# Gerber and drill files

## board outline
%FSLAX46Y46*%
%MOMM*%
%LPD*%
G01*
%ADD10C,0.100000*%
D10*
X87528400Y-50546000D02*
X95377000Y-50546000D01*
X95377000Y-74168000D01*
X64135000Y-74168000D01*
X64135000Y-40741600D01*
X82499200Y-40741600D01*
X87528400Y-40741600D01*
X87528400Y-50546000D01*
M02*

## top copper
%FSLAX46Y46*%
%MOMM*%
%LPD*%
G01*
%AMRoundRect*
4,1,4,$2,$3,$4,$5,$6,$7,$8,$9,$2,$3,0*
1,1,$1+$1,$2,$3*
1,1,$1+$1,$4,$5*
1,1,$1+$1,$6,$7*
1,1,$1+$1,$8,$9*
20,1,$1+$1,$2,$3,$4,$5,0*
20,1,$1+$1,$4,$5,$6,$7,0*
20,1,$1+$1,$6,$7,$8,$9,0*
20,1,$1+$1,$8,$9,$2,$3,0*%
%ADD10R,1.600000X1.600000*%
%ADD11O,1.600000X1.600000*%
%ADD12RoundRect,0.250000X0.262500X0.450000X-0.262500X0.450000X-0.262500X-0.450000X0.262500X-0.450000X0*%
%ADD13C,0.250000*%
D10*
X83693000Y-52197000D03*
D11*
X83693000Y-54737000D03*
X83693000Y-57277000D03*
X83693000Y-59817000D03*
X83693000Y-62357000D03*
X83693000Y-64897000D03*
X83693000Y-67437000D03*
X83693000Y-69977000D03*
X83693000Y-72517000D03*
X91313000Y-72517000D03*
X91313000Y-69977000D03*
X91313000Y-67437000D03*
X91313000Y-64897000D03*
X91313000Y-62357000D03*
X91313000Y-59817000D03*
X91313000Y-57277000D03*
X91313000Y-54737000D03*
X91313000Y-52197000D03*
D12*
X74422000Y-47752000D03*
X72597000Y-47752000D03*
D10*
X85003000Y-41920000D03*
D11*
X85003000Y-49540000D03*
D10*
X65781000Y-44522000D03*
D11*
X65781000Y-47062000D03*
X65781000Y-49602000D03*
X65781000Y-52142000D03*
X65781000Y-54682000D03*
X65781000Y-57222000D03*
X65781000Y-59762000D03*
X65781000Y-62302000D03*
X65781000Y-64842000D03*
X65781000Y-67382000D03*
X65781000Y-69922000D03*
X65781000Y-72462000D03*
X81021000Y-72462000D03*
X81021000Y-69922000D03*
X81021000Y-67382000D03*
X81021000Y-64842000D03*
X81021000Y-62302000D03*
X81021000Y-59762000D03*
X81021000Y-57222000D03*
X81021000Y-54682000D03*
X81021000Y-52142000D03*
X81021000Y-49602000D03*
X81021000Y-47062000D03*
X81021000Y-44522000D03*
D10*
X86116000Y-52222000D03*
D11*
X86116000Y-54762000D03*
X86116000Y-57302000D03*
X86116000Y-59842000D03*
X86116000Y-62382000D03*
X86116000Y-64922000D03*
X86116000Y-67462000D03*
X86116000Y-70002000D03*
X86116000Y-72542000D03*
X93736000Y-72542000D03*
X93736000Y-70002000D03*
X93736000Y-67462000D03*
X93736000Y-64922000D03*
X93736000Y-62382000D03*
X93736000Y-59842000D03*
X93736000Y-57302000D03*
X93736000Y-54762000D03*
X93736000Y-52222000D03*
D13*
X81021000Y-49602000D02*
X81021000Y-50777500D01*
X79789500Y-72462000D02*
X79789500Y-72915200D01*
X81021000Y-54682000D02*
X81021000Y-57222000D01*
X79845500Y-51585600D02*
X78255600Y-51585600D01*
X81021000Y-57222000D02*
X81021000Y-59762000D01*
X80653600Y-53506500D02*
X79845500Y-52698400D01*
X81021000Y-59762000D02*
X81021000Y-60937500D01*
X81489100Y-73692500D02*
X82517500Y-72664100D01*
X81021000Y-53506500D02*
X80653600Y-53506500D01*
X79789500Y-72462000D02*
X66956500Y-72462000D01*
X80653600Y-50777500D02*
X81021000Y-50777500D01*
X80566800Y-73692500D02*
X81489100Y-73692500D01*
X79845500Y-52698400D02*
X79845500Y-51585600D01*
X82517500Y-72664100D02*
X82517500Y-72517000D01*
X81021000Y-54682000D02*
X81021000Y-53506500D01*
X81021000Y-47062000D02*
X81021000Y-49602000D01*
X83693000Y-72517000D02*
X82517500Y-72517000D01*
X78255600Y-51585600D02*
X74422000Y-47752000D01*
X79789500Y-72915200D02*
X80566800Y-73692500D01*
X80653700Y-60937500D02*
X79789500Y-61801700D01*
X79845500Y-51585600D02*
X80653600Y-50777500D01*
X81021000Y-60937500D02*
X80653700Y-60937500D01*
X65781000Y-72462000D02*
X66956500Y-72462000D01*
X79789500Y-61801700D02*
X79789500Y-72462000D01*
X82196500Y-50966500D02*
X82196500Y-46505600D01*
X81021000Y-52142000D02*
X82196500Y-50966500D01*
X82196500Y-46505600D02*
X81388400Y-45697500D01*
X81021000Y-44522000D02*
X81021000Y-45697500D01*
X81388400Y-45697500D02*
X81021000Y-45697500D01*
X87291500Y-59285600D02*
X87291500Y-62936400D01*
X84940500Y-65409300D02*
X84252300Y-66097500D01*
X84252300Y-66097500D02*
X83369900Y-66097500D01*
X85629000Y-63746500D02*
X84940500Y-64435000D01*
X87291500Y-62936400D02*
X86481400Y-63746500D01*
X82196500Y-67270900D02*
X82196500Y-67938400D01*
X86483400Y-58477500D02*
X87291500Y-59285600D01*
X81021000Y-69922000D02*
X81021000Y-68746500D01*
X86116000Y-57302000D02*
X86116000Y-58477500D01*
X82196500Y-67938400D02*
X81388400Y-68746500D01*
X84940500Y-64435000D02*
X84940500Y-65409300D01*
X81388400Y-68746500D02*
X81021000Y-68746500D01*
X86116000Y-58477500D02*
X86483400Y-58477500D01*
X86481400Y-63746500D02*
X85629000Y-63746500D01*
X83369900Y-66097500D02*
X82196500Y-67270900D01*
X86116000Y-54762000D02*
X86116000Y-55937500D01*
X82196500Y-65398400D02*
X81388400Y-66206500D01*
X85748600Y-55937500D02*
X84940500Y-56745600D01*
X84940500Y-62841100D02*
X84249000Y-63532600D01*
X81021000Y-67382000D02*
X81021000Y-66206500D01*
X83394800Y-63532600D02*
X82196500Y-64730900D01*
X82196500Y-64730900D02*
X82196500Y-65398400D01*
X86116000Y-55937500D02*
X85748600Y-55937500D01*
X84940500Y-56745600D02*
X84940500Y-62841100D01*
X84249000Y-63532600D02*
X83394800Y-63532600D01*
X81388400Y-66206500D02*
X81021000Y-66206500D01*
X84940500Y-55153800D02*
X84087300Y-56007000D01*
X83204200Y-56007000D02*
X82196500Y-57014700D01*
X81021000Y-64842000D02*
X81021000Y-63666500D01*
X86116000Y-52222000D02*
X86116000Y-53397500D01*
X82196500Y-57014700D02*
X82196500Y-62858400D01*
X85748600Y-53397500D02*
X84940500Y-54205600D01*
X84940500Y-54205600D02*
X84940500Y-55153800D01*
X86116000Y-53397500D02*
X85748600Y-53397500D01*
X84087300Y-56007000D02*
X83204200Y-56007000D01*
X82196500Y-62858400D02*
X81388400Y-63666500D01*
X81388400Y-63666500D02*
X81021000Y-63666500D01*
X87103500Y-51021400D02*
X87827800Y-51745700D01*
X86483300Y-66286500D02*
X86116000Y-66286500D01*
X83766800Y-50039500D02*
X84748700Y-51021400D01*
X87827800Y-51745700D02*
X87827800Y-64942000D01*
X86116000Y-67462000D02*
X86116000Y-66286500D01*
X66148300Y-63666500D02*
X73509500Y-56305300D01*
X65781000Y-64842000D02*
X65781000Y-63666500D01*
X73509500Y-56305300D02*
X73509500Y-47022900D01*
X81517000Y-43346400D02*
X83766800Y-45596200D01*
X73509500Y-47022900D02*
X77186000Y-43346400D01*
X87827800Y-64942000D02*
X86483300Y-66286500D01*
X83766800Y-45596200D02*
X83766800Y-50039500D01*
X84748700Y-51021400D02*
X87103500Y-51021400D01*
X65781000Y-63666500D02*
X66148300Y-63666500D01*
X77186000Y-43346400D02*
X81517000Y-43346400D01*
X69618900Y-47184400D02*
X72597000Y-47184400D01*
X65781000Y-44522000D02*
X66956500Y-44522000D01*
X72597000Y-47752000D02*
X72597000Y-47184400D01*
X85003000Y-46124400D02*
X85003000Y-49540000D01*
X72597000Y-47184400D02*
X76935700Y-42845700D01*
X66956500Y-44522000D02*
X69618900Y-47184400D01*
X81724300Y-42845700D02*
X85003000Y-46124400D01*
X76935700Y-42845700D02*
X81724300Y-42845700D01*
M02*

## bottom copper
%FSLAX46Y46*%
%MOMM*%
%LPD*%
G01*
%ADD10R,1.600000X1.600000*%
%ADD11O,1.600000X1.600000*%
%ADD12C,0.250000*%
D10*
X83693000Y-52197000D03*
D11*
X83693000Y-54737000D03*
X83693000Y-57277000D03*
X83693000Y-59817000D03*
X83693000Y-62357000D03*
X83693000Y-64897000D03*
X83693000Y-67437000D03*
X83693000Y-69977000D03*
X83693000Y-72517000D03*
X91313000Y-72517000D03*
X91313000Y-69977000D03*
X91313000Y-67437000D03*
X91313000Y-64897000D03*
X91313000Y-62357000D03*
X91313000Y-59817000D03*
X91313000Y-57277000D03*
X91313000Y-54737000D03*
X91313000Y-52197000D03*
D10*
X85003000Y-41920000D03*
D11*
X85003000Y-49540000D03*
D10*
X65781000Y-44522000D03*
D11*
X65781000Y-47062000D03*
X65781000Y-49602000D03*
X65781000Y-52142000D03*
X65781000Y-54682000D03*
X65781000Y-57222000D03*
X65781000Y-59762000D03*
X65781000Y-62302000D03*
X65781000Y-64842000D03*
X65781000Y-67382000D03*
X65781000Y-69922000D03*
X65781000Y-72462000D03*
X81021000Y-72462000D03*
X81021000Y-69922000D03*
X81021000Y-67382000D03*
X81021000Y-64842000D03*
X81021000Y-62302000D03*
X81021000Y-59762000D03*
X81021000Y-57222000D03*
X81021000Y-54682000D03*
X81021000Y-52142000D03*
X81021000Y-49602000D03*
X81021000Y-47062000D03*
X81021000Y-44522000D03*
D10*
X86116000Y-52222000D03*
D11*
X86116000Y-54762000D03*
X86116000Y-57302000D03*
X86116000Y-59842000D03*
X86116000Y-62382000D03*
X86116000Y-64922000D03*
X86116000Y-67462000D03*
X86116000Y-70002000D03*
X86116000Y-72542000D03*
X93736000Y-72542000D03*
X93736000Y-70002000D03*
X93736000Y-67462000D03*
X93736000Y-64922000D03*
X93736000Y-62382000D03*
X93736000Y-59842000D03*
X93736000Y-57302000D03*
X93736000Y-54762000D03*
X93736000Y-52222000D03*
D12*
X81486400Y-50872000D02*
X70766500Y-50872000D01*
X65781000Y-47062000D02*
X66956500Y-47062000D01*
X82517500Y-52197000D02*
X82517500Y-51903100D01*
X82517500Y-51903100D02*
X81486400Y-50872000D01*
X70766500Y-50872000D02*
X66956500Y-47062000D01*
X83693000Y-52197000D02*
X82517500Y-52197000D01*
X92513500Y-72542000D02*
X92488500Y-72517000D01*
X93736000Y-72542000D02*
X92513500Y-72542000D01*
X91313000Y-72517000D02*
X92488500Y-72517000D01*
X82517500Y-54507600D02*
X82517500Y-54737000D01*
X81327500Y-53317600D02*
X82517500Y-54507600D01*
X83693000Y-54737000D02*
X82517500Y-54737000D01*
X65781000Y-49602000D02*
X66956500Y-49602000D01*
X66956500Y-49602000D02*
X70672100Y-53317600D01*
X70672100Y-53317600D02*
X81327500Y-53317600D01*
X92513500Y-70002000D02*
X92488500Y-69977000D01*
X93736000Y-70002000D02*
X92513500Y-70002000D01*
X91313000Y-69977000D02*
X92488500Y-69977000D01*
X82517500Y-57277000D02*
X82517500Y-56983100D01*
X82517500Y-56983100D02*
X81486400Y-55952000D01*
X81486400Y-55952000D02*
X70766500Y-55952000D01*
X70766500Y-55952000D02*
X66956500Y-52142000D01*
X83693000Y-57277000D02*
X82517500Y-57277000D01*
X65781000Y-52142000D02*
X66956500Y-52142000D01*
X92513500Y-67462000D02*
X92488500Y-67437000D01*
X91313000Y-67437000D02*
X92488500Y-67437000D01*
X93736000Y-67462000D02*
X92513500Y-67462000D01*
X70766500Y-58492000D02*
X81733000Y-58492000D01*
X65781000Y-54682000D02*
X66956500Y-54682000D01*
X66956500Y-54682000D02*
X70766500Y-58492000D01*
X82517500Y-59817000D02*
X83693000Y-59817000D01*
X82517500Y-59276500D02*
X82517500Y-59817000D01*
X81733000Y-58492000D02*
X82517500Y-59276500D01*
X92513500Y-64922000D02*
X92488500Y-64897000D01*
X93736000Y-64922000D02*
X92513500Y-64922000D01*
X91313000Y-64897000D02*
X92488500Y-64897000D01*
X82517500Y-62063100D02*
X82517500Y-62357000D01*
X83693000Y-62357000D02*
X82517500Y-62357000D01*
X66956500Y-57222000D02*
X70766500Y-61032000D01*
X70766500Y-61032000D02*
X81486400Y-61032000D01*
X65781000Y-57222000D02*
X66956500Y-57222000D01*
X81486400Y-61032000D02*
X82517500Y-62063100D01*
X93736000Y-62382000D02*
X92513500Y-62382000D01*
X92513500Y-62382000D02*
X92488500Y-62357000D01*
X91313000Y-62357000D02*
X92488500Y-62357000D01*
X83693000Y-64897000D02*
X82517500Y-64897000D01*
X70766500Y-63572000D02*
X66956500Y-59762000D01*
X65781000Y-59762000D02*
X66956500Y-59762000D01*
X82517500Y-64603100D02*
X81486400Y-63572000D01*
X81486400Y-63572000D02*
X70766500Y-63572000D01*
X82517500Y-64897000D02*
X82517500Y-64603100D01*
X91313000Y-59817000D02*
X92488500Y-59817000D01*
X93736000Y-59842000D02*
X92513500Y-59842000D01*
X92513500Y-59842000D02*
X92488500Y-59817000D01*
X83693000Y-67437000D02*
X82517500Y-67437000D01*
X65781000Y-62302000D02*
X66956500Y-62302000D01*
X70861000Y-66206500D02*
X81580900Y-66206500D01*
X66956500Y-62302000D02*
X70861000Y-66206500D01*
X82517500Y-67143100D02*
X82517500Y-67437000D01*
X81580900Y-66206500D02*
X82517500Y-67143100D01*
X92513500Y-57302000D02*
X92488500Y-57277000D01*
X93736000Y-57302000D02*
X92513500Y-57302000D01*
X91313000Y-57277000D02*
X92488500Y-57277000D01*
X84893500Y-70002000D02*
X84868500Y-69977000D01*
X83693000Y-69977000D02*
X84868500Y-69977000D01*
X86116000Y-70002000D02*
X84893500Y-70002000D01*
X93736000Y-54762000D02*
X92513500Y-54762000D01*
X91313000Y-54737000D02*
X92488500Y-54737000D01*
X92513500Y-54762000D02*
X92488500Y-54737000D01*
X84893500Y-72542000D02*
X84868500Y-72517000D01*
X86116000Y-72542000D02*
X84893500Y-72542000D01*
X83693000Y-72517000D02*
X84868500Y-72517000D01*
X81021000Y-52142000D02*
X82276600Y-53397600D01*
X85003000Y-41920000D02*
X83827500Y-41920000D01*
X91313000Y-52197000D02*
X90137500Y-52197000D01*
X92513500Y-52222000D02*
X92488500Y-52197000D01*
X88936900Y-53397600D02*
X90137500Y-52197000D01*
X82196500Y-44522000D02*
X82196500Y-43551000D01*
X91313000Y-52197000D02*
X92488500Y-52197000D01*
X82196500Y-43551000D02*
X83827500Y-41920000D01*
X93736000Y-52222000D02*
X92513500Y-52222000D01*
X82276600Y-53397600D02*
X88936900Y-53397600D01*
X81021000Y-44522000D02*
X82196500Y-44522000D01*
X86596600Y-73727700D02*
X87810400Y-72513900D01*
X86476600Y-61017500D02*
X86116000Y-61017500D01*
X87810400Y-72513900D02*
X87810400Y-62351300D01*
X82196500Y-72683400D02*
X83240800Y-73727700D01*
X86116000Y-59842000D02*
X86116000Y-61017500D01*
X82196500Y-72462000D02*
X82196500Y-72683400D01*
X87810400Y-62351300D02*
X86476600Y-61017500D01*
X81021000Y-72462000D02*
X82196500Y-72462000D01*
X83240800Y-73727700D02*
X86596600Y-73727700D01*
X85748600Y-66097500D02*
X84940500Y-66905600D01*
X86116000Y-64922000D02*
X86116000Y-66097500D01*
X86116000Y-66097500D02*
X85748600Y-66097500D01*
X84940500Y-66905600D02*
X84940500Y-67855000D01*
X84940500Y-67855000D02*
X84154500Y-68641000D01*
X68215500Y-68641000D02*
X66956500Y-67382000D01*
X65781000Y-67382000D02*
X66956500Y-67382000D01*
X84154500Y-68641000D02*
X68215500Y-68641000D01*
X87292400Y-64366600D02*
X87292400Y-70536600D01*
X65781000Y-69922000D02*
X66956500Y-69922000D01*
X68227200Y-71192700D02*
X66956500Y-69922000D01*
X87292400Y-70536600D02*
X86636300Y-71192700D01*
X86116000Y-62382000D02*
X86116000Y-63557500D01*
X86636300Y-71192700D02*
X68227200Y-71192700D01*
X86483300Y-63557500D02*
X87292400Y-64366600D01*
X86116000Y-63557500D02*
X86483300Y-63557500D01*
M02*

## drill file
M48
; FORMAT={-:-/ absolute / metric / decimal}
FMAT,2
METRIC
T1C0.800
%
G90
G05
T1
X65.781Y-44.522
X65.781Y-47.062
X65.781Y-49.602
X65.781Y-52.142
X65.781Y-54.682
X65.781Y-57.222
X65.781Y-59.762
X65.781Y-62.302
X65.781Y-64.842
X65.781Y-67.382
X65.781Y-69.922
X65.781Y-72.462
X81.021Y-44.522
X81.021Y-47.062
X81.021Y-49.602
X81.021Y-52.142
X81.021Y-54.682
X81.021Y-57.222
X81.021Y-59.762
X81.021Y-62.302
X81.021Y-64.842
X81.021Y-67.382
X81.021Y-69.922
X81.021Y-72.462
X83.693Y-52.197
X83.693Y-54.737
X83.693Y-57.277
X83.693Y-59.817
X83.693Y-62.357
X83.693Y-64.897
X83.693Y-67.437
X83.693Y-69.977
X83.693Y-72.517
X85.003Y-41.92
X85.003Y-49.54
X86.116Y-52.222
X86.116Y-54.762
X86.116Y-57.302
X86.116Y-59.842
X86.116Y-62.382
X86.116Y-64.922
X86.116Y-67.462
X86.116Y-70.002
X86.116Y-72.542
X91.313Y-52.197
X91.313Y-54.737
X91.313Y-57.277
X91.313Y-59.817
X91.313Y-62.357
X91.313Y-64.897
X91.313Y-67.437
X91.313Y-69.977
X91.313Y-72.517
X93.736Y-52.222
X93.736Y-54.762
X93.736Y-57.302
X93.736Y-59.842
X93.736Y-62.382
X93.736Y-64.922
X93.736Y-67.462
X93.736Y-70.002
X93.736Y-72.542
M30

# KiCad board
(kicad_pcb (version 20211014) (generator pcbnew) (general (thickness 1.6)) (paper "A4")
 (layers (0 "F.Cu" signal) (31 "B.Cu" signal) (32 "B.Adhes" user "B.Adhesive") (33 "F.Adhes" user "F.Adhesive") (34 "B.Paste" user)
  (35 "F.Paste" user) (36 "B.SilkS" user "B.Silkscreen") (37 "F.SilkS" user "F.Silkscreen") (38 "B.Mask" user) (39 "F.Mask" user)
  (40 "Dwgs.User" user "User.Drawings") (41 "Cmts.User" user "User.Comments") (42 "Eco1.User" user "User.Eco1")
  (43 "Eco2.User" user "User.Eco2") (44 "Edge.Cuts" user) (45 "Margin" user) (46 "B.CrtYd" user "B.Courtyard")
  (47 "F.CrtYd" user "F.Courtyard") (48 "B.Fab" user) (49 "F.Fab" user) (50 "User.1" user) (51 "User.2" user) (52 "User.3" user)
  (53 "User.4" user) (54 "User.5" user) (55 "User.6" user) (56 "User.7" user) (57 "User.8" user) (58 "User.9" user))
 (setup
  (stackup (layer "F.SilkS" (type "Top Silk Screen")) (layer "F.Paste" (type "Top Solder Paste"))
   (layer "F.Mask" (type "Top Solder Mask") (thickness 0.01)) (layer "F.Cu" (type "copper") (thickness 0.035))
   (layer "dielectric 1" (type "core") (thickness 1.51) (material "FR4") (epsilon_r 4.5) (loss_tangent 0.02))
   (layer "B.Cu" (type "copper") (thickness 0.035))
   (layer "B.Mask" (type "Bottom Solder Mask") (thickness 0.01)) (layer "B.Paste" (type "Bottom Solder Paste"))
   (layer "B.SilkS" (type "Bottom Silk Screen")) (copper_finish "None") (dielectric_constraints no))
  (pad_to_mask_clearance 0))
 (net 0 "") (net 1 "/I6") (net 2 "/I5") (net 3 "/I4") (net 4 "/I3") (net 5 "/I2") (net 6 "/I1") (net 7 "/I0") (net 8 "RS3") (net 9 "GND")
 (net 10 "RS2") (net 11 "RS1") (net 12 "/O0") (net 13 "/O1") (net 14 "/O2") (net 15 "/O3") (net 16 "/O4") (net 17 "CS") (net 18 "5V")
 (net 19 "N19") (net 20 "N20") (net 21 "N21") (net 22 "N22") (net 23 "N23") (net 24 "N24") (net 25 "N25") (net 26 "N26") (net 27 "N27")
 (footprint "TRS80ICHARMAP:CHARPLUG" (layer "F.Cu") (at 83.693 52.197)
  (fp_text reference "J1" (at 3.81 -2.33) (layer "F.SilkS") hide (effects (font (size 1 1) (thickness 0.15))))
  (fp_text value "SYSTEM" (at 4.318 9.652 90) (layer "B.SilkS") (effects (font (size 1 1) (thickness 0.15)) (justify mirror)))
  (pad "1" thru_hole rect (at 0 0) (size 1.6 1.6) (drill 0.8) (layers *.Cu *.Mask) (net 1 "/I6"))
  (pad "2" thru_hole oval (at 0 2.54) (size 1.6 1.6) (drill 0.8) (layers *.Cu *.Mask) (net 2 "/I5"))
  (pad "3" thru_hole oval (at 0 5.08) (size 1.6 1.6) (drill 0.8) (layers *.Cu *.Mask) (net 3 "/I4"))
  (pad "4" thru_hole oval (at 0 7.62) (size 1.6 1.6) (drill 0.8) (layers *.Cu *.Mask) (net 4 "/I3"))
  (pad "5" thru_hole oval (at 0 10.16) (size 1.6 1.6) (drill 0.8) (layers *.Cu *.Mask) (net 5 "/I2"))
  (pad "6" thru_hole oval (at 0 12.7) (size 1.6 1.6) (drill 0.8) (layers *.Cu *.Mask) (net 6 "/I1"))
  (pad "7" thru_hole oval (at 0 15.24) (size 1.6 1.6) (drill 0.8) (layers *.Cu *.Mask) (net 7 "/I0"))
  (pad "8" thru_hole oval (at 0 17.78) (size 1.6 1.6) (drill 0.8) (layers *.Cu *.Mask) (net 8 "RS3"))
  (pad "9" thru_hole oval (at 0 20.32) (size 1.6 1.6) (drill 0.8) (layers *.Cu *.Mask) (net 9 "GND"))
  (pad "10" thru_hole oval (at 7.62 20.32) (size 1.6 1.6) (drill 0.8) (layers *.Cu *.Mask) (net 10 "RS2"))
  (pad "11" thru_hole oval (at 7.62 17.78) (size 1.6 1.6) (drill 0.8) (layers *.Cu *.Mask) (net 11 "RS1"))
  (pad "12" thru_hole oval (at 7.62 15.24) (size 1.6 1.6) (drill 0.8) (layers *.Cu *.Mask) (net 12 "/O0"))
  (pad "13" thru_hole oval (at 7.62 12.7) (size 1.6 1.6) (drill 0.8) (layers *.Cu *.Mask) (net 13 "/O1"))
  (pad "14" thru_hole oval (at 7.62 10.16) (size 1.6 1.6) (drill 0.8) (layers *.Cu *.Mask) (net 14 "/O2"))
  (pad "15" thru_hole oval (at 7.62 7.62) (size 1.6 1.6) (drill 0.8) (layers *.Cu *.Mask) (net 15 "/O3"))
  (pad "16" thru_hole oval (at 7.62 5.08) (size 1.6 1.6) (drill 0.8) (layers *.Cu *.Mask) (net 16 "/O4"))
  (pad "17" thru_hole oval (at 7.62 2.54) (size 1.6 1.6) (drill 0.8) (layers *.Cu *.Mask) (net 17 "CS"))
  (pad "18" thru_hole oval (at 7.62 0) (size 1.6 1.6) (drill 0.8) (layers *.Cu *.Mask) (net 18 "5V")))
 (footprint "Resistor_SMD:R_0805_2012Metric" (layer "F.Cu") (at 73.5095 47.752 180)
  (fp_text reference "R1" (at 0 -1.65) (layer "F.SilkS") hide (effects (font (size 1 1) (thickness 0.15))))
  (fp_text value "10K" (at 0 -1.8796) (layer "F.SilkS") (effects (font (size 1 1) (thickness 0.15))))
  (pad "1" smd roundrect locked (at -0.9125 0 180) (size 1.025 1.4) (layers "F.Cu" "F.Paste" "F.Mask") (roundrect_rratio 0.243902439)
   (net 9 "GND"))
  (pad "2" smd roundrect locked (at 0.9125 0 180) (size 1.025 1.4) (layers "F.Cu" "F.Paste" "F.Mask") (roundrect_rratio 0.243902439)
   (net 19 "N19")))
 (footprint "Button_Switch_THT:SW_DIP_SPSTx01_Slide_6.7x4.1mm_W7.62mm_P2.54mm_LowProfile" (layer "F.Cu") (at 85.003 41.92 -90)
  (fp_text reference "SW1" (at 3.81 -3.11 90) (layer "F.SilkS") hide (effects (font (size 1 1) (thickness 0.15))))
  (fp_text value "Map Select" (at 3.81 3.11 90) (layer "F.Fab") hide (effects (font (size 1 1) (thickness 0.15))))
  (pad "1" thru_hole rect locked (at 0 0 270) (size 1.6 1.6) (drill 0.8) (layers *.Cu *.Mask) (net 18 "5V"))
  (pad "2" thru_hole oval locked (at 7.62 0 270) (size 1.6 1.6) (drill 0.8) (layers *.Cu *.Mask) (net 19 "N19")))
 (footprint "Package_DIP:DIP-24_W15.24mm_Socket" (layer "F.Cu") (at 65.781 44.522)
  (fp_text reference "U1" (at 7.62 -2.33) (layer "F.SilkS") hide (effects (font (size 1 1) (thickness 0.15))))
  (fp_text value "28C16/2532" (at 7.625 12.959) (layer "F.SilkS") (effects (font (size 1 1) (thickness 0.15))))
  (pad "1" thru_hole rect locked (at 0 0) (size 1.6 1.6) (drill 0.8) (layers *.Cu *.Mask) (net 19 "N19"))
  (pad "2" thru_hole oval locked (at 0 2.54) (size 1.6 1.6) (drill 0.8) (layers *.Cu *.Mask) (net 1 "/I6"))
  (pad "3" thru_hole oval locked (at 0 5.08) (size 1.6 1.6) (drill 0.8) (layers *.Cu *.Mask) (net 2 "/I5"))
  (pad "4" thru_hole oval locked (at 0 7.62) (size 1.6 1.6) (drill 0.8) (layers *.Cu *.Mask) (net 3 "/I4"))
  (pad "5" thru_hole oval locked (at 0 10.16) (size 1.6 1.6) (drill 0.8) (layers *.Cu *.Mask) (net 4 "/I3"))
  (pad "6" thru_hole oval locked (at 0 12.7) (size 1.6 1.6) (drill 0.8) (layers *.Cu *.Mask) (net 5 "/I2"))
  (pad "7" thru_hole oval locked (at 0 15.24) (size 1.6 1.6) (drill 0.8) (layers *.Cu *.Mask) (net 6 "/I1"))
  (pad "8" thru_hole oval locked (at 0 17.78) (size 1.6 1.6) (drill 0.8) (layers *.Cu *.Mask) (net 7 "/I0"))
  (pad "9" thru_hole oval locked (at 0 20.32) (size 1.6 1.6) (drill 0.8) (layers *.Cu *.Mask) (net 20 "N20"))
  (pad "10" thru_hole oval locked (at 0 22.86) (size 1.6 1.6) (drill 0.8) (layers *.Cu *.Mask) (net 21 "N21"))
  (pad "11" thru_hole oval locked (at 0 25.4) (size 1.6 1.6) (drill 0.8) (layers *.Cu *.Mask) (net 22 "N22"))
  (pad "12" thru_hole oval locked (at 0 27.94) (size 1.6 1.6) (drill 0.8) (layers *.Cu *.Mask) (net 9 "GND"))
  (pad "13" thru_hole oval locked (at 15.24 27.94) (size 1.6 1.6) (drill 0.8) (layers *.Cu *.Mask) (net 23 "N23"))
  (pad "14" thru_hole oval locked (at 15.24 25.4) (size 1.6 1.6) (drill 0.8) (layers *.Cu *.Mask) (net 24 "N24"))
  (pad "15" thru_hole oval locked (at 15.24 22.86) (size 1.6 1.6) (drill 0.8) (layers *.Cu *.Mask) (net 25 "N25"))
  (pad "16" thru_hole oval locked (at 15.24 20.32) (size 1.6 1.6) (drill 0.8) (layers *.Cu *.Mask) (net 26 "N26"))
  (pad "17" thru_hole oval locked (at 15.24 17.78) (size 1.6 1.6) (drill 0.8) (layers *.Cu *.Mask) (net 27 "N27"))
  (pad "18" thru_hole oval locked (at 15.24 15.24) (size 1.6 1.6) (drill 0.8) (layers *.Cu *.Mask) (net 9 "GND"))
  (pad "19" thru_hole oval locked (at 15.24 12.7) (size 1.6 1.6) (drill 0.8) (layers *.Cu *.Mask) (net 9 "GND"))
  (pad "20" thru_hole oval locked (at 15.24 10.16) (size 1.6 1.6) (drill 0.8) (layers *.Cu *.Mask) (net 9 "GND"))
  (pad "21" thru_hole oval locked (at 15.24 7.62) (size 1.6 1.6) (drill 0.8) (layers *.Cu *.Mask) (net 18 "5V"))
  (pad "22" thru_hole oval locked (at 15.24 5.08) (size 1.6 1.6) (drill 0.8) (layers *.Cu *.Mask) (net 9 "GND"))
  (pad "23" thru_hole oval locked (at 15.24 2.54) (size 1.6 1.6) (drill 0.8) (layers *.Cu *.Mask) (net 9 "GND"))
  (pad "24" thru_hole oval locked (at 15.24 0) (size 1.6 1.6) (drill 0.8) (layers *.Cu *.Mask) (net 18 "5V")))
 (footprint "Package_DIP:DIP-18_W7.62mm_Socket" (layer "F.Cu") (at 86.116 52.222)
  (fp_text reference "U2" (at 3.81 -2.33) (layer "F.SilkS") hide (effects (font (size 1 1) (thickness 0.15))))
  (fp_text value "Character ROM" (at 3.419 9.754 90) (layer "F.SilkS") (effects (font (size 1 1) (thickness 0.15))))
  (pad "1" thru_hole rect locked (at 0 0) (size 1.6 1.6) (drill 0.8) (layers *.Cu *.Mask) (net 26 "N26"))
  (pad "2" thru_hole oval locked (at 0 2.54) (size 1.6 1.6) (drill 0.8) (layers *.Cu *.Mask) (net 25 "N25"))
  (pad "3" thru_hole oval locked (at 0 5.08) (size 1.6 1.6) (drill 0.8) (layers *.Cu *.Mask) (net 24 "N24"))
  (pad "4" thru_hole oval locked (at 0 7.62) (size 1.6 1.6) (drill 0.8) (layers *.Cu *.Mask) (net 23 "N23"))
  (pad "5" thru_hole oval locked (at 0 10.16) (size 1.6 1.6) (drill 0.8) (layers *.Cu *.Mask) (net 22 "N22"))
  (pad "6" thru_hole oval locked (at 0 12.7) (size 1.6 1.6) (drill 0.8) (layers *.Cu *.Mask) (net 21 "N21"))
  (pad "7" thru_hole oval locked (at 0 15.24) (size 1.6 1.6) (drill 0.8) (layers *.Cu *.Mask) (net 20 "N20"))
  (pad "8" thru_hole oval locked (at 0 17.78) (size 1.6 1.6) (drill 0.8) (layers *.Cu *.Mask) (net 8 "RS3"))
  (pad "9" thru_hole oval locked (at 0 20.32) (size 1.6 1.6) (drill 0.8) (layers *.Cu *.Mask) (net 9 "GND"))
  (pad "10" thru_hole oval locked (at 7.62 20.32) (size 1.6 1.6) (drill 0.8) (layers *.Cu *.Mask) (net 10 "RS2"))
  (pad "11" thru_hole oval locked (at 7.62 17.78) (size 1.6 1.6) (drill 0.8) (layers *.Cu *.Mask) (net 11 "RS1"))
  (pad "12" thru_hole oval locked (at 7.62 15.24) (size 1.6 1.6) (drill 0.8) (layers *.Cu *.Mask) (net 12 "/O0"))
  (pad "13" thru_hole oval locked (at 7.62 12.7) (size 1.6 1.6) (drill 0.8) (layers *.Cu *.Mask) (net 13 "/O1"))
  (pad "14" thru_hole oval locked (at 7.62 10.16) (size 1.6 1.6) (drill 0.8) (layers *.Cu *.Mask) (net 14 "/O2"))
  (pad "15" thru_hole oval locked (at 7.62 7.62) (size 1.6 1.6) (drill 0.8) (layers *.Cu *.Mask) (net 15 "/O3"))
  (pad "16" thru_hole oval locked (at 7.62 5.08) (size 1.6 1.6) (drill 0.8) (layers *.Cu *.Mask) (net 16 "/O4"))
  (pad "17" thru_hole oval locked (at 7.62 2.54) (size 1.6 1.6) (drill 0.8) (layers *.Cu *.Mask) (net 17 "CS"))
  (pad "18" thru_hole oval locked (at 7.62 0) (size 1.6 1.6) (drill 0.8) (layers *.Cu *.Mask) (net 18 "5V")))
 (gr_poly
  (pts (xy 87.5284 50.546) (xy 95.377 50.546) (xy 95.377 74.168) (xy 64.135 74.168) (xy 64.135 40.7416) (xy 82.4992 40.7416)
   (xy 87.5284 40.7416))
  (layer "Edge.Cuts") (width 0.1) (fill none))
 (segment (start 81.4864 50.872) (end 70.7665 50.872) (width 0.25) (layer "B.Cu") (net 1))
 (segment (start 65.781 47.062) (end 66.9565 47.062) (width 0.25) (layer "B.Cu") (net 1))
 (segment (start 82.5175 52.197) (end 82.5175 51.9031) (width 0.25) (layer "B.Cu") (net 1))
 (segment (start 82.5175 51.9031) (end 81.4864 50.872) (width 0.25) (layer "B.Cu") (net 1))
 (segment (start 70.7665 50.872) (end 66.9565 47.062) (width 0.25) (layer "B.Cu") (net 1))
 (segment (start 83.693 52.197) (end 82.5175 52.197) (width 0.25) (layer "B.Cu") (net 1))
 (segment (start 92.5135 72.542) (end 92.4885 72.517) (width 0.25) (layer "B.Cu") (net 10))
 (segment (start 93.736 72.542) (end 92.5135 72.542) (width 0.25) (layer "B.Cu") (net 10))
 (segment (start 91.313 72.517) (end 92.4885 72.517) (width 0.25) (layer "B.Cu") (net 10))
 (segment (start 82.5175 54.5076) (end 82.5175 54.737) (width 0.25) (layer "B.Cu") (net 2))
 (segment (start 81.3275 53.3176) (end 82.5175 54.5076) (width 0.25) (layer "B.Cu") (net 2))
 (segment (start 83.693 54.737) (end 82.5175 54.737) (width 0.25) (layer "B.Cu") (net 2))
 (segment (start 65.781 49.602) (end 66.9565 49.602) (width 0.25) (layer "B.Cu") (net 2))
 (segment (start 66.9565 49.602) (end 70.6721 53.3176) (width 0.25) (layer "B.Cu") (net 2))
 (segment (start 70.6721 53.3176) (end 81.3275 53.3176) (width 0.25) (layer "B.Cu") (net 2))
 (segment (start 92.5135 70.002) (end 92.4885 69.977) (width 0.25) (layer "B.Cu") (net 11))
 (segment (start 93.736 70.002) (end 92.5135 70.002) (width 0.25) (layer "B.Cu") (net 11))
 (segment (start 91.313 69.977) (end 92.4885 69.977) (width 0.25) (layer "B.Cu") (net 11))
 (segment (start 82.5175 57.277) (end 82.5175 56.9831) (width 0.25) (layer "B.Cu") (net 3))
 (segment (start 82.5175 56.9831) (end 81.4864 55.952) (width 0.25) (layer "B.Cu") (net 3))
 (segment (start 81.4864 55.952) (end 70.7665 55.952) (width 0.25) (layer "B.Cu") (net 3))
 (segment (start 70.7665 55.952) (end 66.9565 52.142) (width 0.25) (layer "B.Cu") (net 3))
 (segment (start 83.693 57.277) (end 82.5175 57.277) (width 0.25) (layer "B.Cu") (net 3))
 (segment (start 65.781 52.142) (end 66.9565 52.142) (width 0.25) (layer "B.Cu") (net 3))
 (segment (start 92.5135 67.462) (end 92.4885 67.437) (width 0.25) (layer "B.Cu") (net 12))
 (segment (start 91.313 67.437) (end 92.4885 67.437) (width 0.25) (layer "B.Cu") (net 12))
 (segment (start 93.736 67.462) (end 92.5135 67.462) (width 0.25) (layer "B.Cu") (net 12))
 (segment (start 70.7665 58.492) (end 81.733 58.492) (width 0.25) (layer "B.Cu") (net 4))
 (segment (start 65.781 54.682) (end 66.9565 54.682) (width 0.25) (layer "B.Cu") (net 4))
 (segment (start 66.9565 54.682) (end 70.7665 58.492) (width 0.25) (layer "B.Cu") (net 4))
 (segment (start 82.5175 59.817) (end 83.693 59.817) (width 0.25) (layer "B.Cu") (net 4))
 (segment (start 82.5175 59.2765) (end 82.5175 59.817) (width 0.25) (layer "B.Cu") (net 4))
 (segment (start 81.733 58.492) (end 82.5175 59.2765) (width 0.25) (layer "B.Cu") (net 4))
 (segment (start 92.5135 64.922) (end 92.4885 64.897) (width 0.25) (layer "B.Cu") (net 13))
 (segment (start 93.736 64.922) (end 92.5135 64.922) (width 0.25) (layer "B.Cu") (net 13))
 (segment (start 91.313 64.897) (end 92.4885 64.897) (width 0.25) (layer "B.Cu") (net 13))
 (segment (start 82.5175 62.0631) (end 82.5175 62.357) (width 0.25) (layer "B.Cu") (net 5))
 (segment (start 83.693 62.357) (end 82.5175 62.357) (width 0.25) (layer "B.Cu") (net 5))
 (segment (start 66.9565 57.222) (end 70.7665 61.032) (width 0.25) (layer "B.Cu") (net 5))
 (segment (start 70.7665 61.032) (end 81.4864 61.032) (width 0.25) (layer "B.Cu") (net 5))
 (segment (start 65.781 57.222) (end 66.9565 57.222) (width 0.25) (layer "B.Cu") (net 5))
 (segment (start 81.4864 61.032) (end 82.5175 62.0631) (width 0.25) (layer "B.Cu") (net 5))
 (segment (start 93.736 62.382) (end 92.5135 62.382) (width 0.25) (layer "B.Cu") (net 14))
 (segment (start 92.5135 62.382) (end 92.4885 62.357) (width 0.25) (layer "B.Cu") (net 14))
 (segment (start 91.313 62.357) (end 92.4885 62.357) (width 0.25) (layer "B.Cu") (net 14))
 (segment (start 83.693 64.897) (end 82.5175 64.897) (width 0.25) (layer "B.Cu") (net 6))
 (segment (start 70.7665 63.572) (end 66.9565 59.762) (width 0.25) (layer "B.Cu") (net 6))
 (segment (start 65.781 59.762) (end 66.9565 59.762) (width 0.25) (layer "B.Cu") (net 6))
 (segment (start 82.5175 64.6031) (end 81.4864 63.572) (width 0.25) (layer "B.Cu") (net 6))
 (segment (start 81.4864 63.572) (end 70.7665 63.572) (width 0.25) (layer "B.Cu") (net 6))
 (segment (start 82.5175 64.897) (end 82.5175 64.6031) (width 0.25) (layer "B.Cu") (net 6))
 (segment (start 91.313 59.817) (end 92.4885 59.817) (width 0.25) (layer "B.Cu") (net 15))
 (segment (start 93.736 59.842) (end 92.5135 59.842) (width 0.25) (layer "B.Cu") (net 15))
 (segment (start 92.5135 59.842) (end 92.4885 59.817) (width 0.25) (layer "B.Cu") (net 15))
 (segment (start 83.693 67.437) (end 82.5175 67.437) (width 0.25) (layer "B.Cu") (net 7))
 (segment (start 65.781 62.302) (end 66.9565 62.302) (width 0.25) (layer "B.Cu") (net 7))
 (segment (start 70.861 66.2065) (end 81.5809 66.2065) (width 0.25) (layer "B.Cu") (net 7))
 (segment (start 66.9565 62.302) (end 70.861 66.2065) (width 0.25) (layer "B.Cu") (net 7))
 (segment (start 82.5175 67.1431) (end 82.5175 67.437) (width 0.25) (layer "B.Cu") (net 7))
 (segment (start 81.5809 66.2065) (end 82.5175 67.1431) (width 0.25) (layer "B.Cu") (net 7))
 (segment (start 92.5135 57.302) (end 92.4885 57.277) (width 0.25) (layer "B.Cu") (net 16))
 (segment (start 93.736 57.302) (end 92.5135 57.302) (width 0.25) (layer "B.Cu") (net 16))
 (segment (start 91.313 57.277) (end 92.4885 57.277) (width 0.25) (layer "B.Cu") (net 16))
 (segment (start 84.8935 70.002) (end 84.8685 69.977) (width 0.25) (layer "B.Cu") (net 8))
 (segment (start 83.693 69.977) (end 84.8685 69.977) (width 0.25) (layer "B.Cu") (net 8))
 (segment (start 86.116 70.002) (end 84.8935 70.002) (width 0.25) (layer "B.Cu") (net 8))
 (segment (start 93.736 54.762) (end 92.5135 54.762) (width 0.25) (layer "B.Cu") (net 17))
 (segment (start 91.313 54.737) (end 92.4885 54.737) (width 0.25) (layer "B.Cu") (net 17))
 (segment (start 92.5135 54.762) (end 92.4885 54.737) (width 0.25) (layer "B.Cu") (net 17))
 (segment (start 81.021 49.602) (end 81.021 50.7775) (width 0.25) (layer "F.Cu") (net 9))
 (segment (start 79.7895 72.462) (end 79.7895 72.9152) (width 0.25) (layer "F.Cu") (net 9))
 (segment (start 81.021 54.682) (end 81.021 57.222) (width 0.25) (layer "F.Cu") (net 9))
 (segment (start 79.8455 51.5856) (end 78.2556 51.5856) (width 0.25) (layer "F.Cu") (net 9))
 (segment (start 81.021 57.222) (end 81.021 59.762) (width 0.25) (layer "F.Cu") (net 9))
 (segment (start 80.6536 53.5065) (end 79.8455 52.6984) (width 0.25) (layer "F.Cu") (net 9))
 (segment (start 81.021 59.762) (end 81.021 60.9375) (width 0.25) (layer "F.Cu") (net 9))
 (segment (start 81.4891 73.6925) (end 82.5175 72.6641) (width 0.25) (layer "F.Cu") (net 9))
 (segment (start 81.021 53.5065) (end 80.6536 53.5065) (width 0.25) (layer "F.Cu") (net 9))
 (segment (start 79.7895 72.462) (end 66.9565 72.462) (width 0.25) (layer "F.Cu") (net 9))
 (segment (start 80.6536 50.7775) (end 81.021 50.7775) (width 0.25) (layer "F.Cu") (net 9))
 (segment (start 80.5668 73.6925) (end 81.4891 73.6925) (width 0.25) (layer "F.Cu") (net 9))
 (segment (start 79.8455 52.6984) (end 79.8455 51.5856) (width 0.25) (layer "F.Cu") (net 9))
 (segment (start 82.5175 72.6641) (end 82.5175 72.517) (width 0.25) (layer "F.Cu") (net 9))
 (segment (start 81.021 54.682) (end 81.021 53.5065) (width 0.25) (layer "F.Cu") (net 9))
 (segment (start 81.021 47.062) (end 81.021 49.602) (width 0.25) (layer "F.Cu") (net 9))
 (segment (start 83.693 72.517) (end 82.5175 72.517) (width 0.25) (layer "F.Cu") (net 9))
 (segment (start 78.2556 51.5856) (end 74.422 47.752) (width 0.25) (layer "F.Cu") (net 9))
 (segment (start 79.7895 72.9152) (end 80.5668 73.6925) (width 0.25) (layer "F.Cu") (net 9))
 (segment (start 80.6537 60.9375) (end 79.7895 61.8017) (width 0.25) (layer "F.Cu") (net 9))
 (segment (start 79.8455 51.5856) (end 80.6536 50.7775) (width 0.25) (layer "F.Cu") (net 9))
 (segment (start 81.021 60.9375) (end 80.6537 60.9375) (width 0.25) (layer "F.Cu") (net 9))
 (segment (start 65.781 72.462) (end 66.9565 72.462) (width 0.25) (layer "F.Cu") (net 9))
 (segment (start 79.7895 61.8017) (end 79.7895 72.462) (width 0.25) (layer "F.Cu") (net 9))
 (segment (start 84.8935 72.542) (end 84.8685 72.517) (width 0.25) (layer "B.Cu") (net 9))
 (segment (start 86.116 72.542) (end 84.8935 72.542) (width 0.25) (layer "B.Cu") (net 9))
 (segment (start 83.693 72.517) (end 84.8685 72.517) (width 0.25) (layer "B.Cu") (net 9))
 (segment (start 82.1965 50.9665) (end 82.1965 46.5056) (width 0.25) (layer "F.Cu") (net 18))
 (segment (start 81.021 52.142) (end 82.1965 50.9665) (width 0.25) (layer "F.Cu") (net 18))
 (segment (start 82.1965 46.5056) (end 81.3884 45.6975) (width 0.25) (layer "F.Cu") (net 18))
 (segment (start 81.021 44.522) (end 81.021 45.6975) (width 0.25) (layer "F.Cu") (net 18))
 (segment (start 81.3884 45.6975) (end 81.021 45.6975) (width 0.25) (layer "F.Cu") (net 18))
 (segment (start 81.021 52.142) (end 82.2766 53.3976) (width 0.25) (layer "B.Cu") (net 18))
 (segment (start 85.003 41.92) (end 83.8275 41.92) (width 0.25) (layer "B.Cu") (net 18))
 (segment (start 91.313 52.197) (end 90.1375 52.197) (width 0.25) (layer "B.Cu") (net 18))
 (segment (start 92.5135 52.222) (end 92.4885 52.197) (width 0.25) (layer "B.Cu") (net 18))
 (segment (start 88.9369 53.3976) (end 90.1375 52.197) (width 0.25) (layer "B.Cu") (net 18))
 (segment (start 82.1965 44.522) (end 82.1965 43.551) (width 0.25) (layer "B.Cu") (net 18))
 (segment (start 91.313 52.197) (end 92.4885 52.197) (width 0.25) (layer "B.Cu") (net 18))
 (segment (start 82.1965 43.551) (end 83.8275 41.92) (width 0.25) (layer "B.Cu") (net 18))
 (segment (start 93.736 52.222) (end 92.5135 52.222) (width 0.25) (layer "B.Cu") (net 18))
 (segment (start 82.2766 53.3976) (end 88.9369 53.3976) (width 0.25) (layer "B.Cu") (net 18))
 (segment (start 81.021 44.522) (end 82.1965 44.522) (width 0.25) (layer "B.Cu") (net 18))
 (segment (start 86.5966 73.7277) (end 87.8104 72.5139) (width 0.25) (layer "B.Cu") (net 23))
 (segment (start 86.4766 61.0175) (end 86.116 61.0175) (width 0.25) (layer "B.Cu") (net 23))
 (segment (start 87.8104 72.5139) (end 87.8104 62.3513) (width 0.25) (layer "B.Cu") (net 23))
 (segment (start 82.1965 72.6834) (end 83.2408 73.7277) (width 0.25) (layer "B.Cu") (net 23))
 (segment (start 86.116 59.842) (end 86.116 61.0175) (width 0.25) (layer "B.Cu") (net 23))
 (segment (start 82.1965 72.462) (end 82.1965 72.6834) (width 0.25) (layer "B.Cu") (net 23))
 (segment (start 87.8104 62.3513) (end 86.4766 61.0175) (width 0.25) (layer "B.Cu") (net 23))
 (segment (start 81.021 72.462) (end 82.1965 72.462) (width 0.25) (layer "B.Cu") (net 23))
 (segment (start 83.2408 73.7277) (end 86.5966 73.7277) (width 0.25) (layer "B.Cu") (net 23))
 (segment (start 87.2915 59.2856) (end 87.2915 62.9364) (width 0.25) (layer "F.Cu") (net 24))
 (segment (start 84.9405 65.4093) (end 84.2523 66.0975) (width 0.25) (layer "F.Cu") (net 24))
 (segment (start 84.2523 66.0975) (end 83.3699 66.0975) (width 0.25) (layer "F.Cu") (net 24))
 (segment (start 85.629 63.7465) (end 84.9405 64.435) (width 0.25) (layer "F.Cu") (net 24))
 (segment (start 87.2915 62.9364) (end 86.4814 63.7465) (width 0.25) (layer "F.Cu") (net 24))
 (segment (start 82.1965 67.2709) (end 82.1965 67.9384) (width 0.25) (layer "F.Cu") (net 24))
 (segment (start 86.4834 58.4775) (end 87.2915 59.2856) (width 0.25) (layer "F.Cu") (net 24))
 (segment (start 81.021 69.922) (end 81.021 68.7465) (width 0.25) (layer "F.Cu") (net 24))
 (segment (start 86.116 57.302) (end 86.116 58.4775) (width 0.25) (layer "F.Cu") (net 24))
 (segment (start 82.1965 67.9384) (end 81.3884 68.7465) (width 0.25) (layer "F.Cu") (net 24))
 (segment (start 84.9405 64.435) (end 84.9405 65.4093) (width 0.25) (layer "F.Cu") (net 24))
 (segment (start 81.3884 68.7465) (end 81.021 68.7465) (width 0.25) (layer "F.Cu") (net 24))
 (segment (start 86.116 58.4775) (end 86.4834 58.4775) (width 0.25) (layer "F.Cu") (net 24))
 (segment (start 86.4814 63.7465) (end 85.629 63.7465) (width 0.25) (layer "F.Cu") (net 24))
 (segment (start 83.3699 66.0975) (end 82.1965 67.2709) (width 0.25) (layer "F.Cu") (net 24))
 (segment (start 86.116 54.762) (end 86.116 55.9375) (width 0.25) (layer "F.Cu") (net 25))
 (segment (start 82.1965 65.3984) (end 81.3884 66.2065) (width 0.25) (layer "F.Cu") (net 25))
 (segment (start 85.7486 55.9375) (end 84.9405 56.7456) (width 0.25) (layer "F.Cu") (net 25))
 (segment (start 84.9405 62.8411) (end 84.249 63.5326) (width 0.25) (layer "F.Cu") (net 25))
 (segment (start 81.021 67.382) (end 81.021 66.2065) (width 0.25) (layer "F.Cu") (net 25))
 (segment (start 83.3948 63.5326) (end 82.1965 64.7309) (width 0.25) (layer "F.Cu") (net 25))
 (segment (start 82.1965 64.7309) (end 82.1965 65.3984) (width 0.25) (layer "F.Cu") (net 25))
 (segment (start 86.116 55.9375) (end 85.7486 55.9375) (width 0.25) (layer "F.Cu") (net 25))
 (segment (start 84.9405 56.7456) (end 84.9405 62.8411) (width 0.25) (layer "F.Cu") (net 25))
 (segment (start 84.249 63.5326) (end 83.3948 63.5326) (width 0.25) (layer "F.Cu") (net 25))
 (segment (start 81.3884 66.2065) (end 81.021 66.2065) (width 0.25) (layer "F.Cu") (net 25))
 (segment (start 84.9405 55.1538) (end 84.0873 56.007) (width 0.25) (layer "F.Cu") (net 26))
 (segment (start 83.2042 56.007) (end 82.1965 57.0147) (width 0.25) (layer "F.Cu") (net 26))
 (segment (start 81.021 64.842) (end 81.021 63.6665) (width 0.25) (layer "F.Cu") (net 26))
 (segment (start 86.116 52.222) (end 86.116 53.3975) (width 0.25) (layer "F.Cu") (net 26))
 (segment (start 82.1965 57.0147) (end 82.1965 62.8584) (width 0.25) (layer "F.Cu") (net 26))
 (segment (start 85.7486 53.3975) (end 84.9405 54.2056) (width 0.25) (layer "F.Cu") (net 26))
 (segment (start 84.9405 54.2056) (end 84.9405 55.1538) (width 0.25) (layer "F.Cu") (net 26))
 (segment (start 86.116 53.3975) (end 85.7486 53.3975) (width 0.25) (layer "F.Cu") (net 26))
 (segment (start 84.0873 56.007) (end 83.2042 56.007) (width 0.25) (layer "F.Cu") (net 26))
 (segment (start 82.1965 62.8584) (end 81.3884 63.6665) (width 0.25) (layer "F.Cu") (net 26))
 (segment (start 81.3884 63.6665) (end 81.021 63.6665) (width 0.25) (layer "F.Cu") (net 26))
 (segment (start 87.1035 51.0214) (end 87.8278 51.7457) (width 0.25) (layer "F.Cu") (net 20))
 (segment (start 86.4833 66.2865) (end 86.116 66.2865) (width 0.25) (layer "F.Cu") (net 20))
 (segment (start 83.7668 50.0395) (end 84.7487 51.0214) (width 0.25) (layer "F.Cu") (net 20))
 (segment (start 87.8278 51.7457) (end 87.8278 64.942) (width 0.25) (layer "F.Cu") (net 20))
 (segment (start 86.116 67.462) (end 86.116 66.2865) (width 0.25) (layer "F.Cu") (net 20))
 (segment (start 66.1483 63.6665) (end 73.5095 56.3053) (width 0.25) (layer "F.Cu") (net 20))
 (segment (start 65.781 64.842) (end 65.781 63.6665) (width 0.25) (layer "F.Cu") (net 20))
 (segment (start 73.5095 56.3053) (end 73.5095 47.0229) (width 0.25) (layer "F.Cu") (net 20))
 (segment (start 81.517 43.3464) (end 83.7668 45.5962) (width 0.25) (layer "F.Cu") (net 20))
 (segment (start 73.5095 47.0229) (end 77.186 43.3464) (width 0.25) (layer "F.Cu") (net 20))
 (segment (start 87.8278 64.942) (end 86.4833 66.2865) (width 0.25) (layer "F.Cu") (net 20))
 (segment (start 83.7668 45.5962) (end 83.7668 50.0395) (width 0.25) (layer "F.Cu") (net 20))
 (segment (start 84.7487 51.0214) (end 87.1035 51.0214) (width 0.25) (layer "F.Cu") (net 20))
 (segment (start 65.781 63.6665) (end 66.1483 63.6665) (width 0.25) (layer "F.Cu") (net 20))
 (segment (start 77.186 43.3464) (end 81.517 43.3464) (width 0.25) (layer "F.Cu") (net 20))
 (segment (start 85.7486 66.0975) (end 84.9405 66.9056) (width 0.25) (layer "B.Cu") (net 21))
 (segment (start 86.116 64.922) (end 86.116 66.0975) (width 0.25) (layer "B.Cu") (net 21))
 (segment (start 86.116 66.0975) (end 85.7486 66.0975) (width 0.25) (layer "B.Cu") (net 21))
 (segment (start 84.9405 66.9056) (end 84.9405 67.855) (width 0.25) (layer "B.Cu") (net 21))
 (segment (start 84.9405 67.855) (end 84.1545 68.641) (width 0.25) (layer "B.Cu") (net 21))
 (segment (start 68.2155 68.641) (end 66.9565 67.382) (width 0.25) (layer "B.Cu") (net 21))
 (segment (start 65.781 67.382) (end 66.9565 67.382) (width 0.25) (layer "B.Cu") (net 21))
 (segment (start 84.1545 68.641) (end 68.2155 68.641) (width 0.25) (layer "B.Cu") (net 21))
 (segment (start 87.2924 64.3666) (end 87.2924 70.5366) (width 0.25) (layer "B.Cu") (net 22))
 (segment (start 65.781 69.922) (end 66.9565 69.922) (width 0.25) (layer "B.Cu") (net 22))
 (segment (start 68.2272 71.1927) (end 66.9565 69.922) (width 0.25) (layer "B.Cu") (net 22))
 (segment (start 87.2924 70.5366) (end 86.6363 71.1927) (width 0.25) (layer "B.Cu") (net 22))
 (segment (start 86.116 62.382) (end 86.116 63.5575) (width 0.25) (layer "B.Cu") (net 22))
 (segment (start 86.6363 71.1927) (end 68.2272 71.1927) (width 0.25) (layer "B.Cu") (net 22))
 (segment (start 86.4833 63.5575) (end 87.2924 64.3666) (width 0.25) (layer "B.Cu") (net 22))
 (segment (start 86.116 63.5575) (end 86.4833 63.5575) (width 0.25) (layer "B.Cu") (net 22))
 (segment (start 69.6189 47.1844) (end 72.597 47.1844) (width 0.25) (layer "F.Cu") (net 19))
 (segment (start 65.781 44.522) (end 66.9565 44.522) (width 0.25) (layer "F.Cu") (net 19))
 (segment (start 72.597 47.752) (end 72.597 47.1844) (width 0.25) (layer "F.Cu") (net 19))
 (segment (start 85.003 46.1244) (end 85.003 49.54) (width 0.25) (layer "F.Cu") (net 19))
 (segment (start 72.597 47.1844) (end 76.9357 42.8457) (width 0.25) (layer "F.Cu") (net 19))
 (segment (start 66.9565 44.522) (end 69.6189 47.1844) (width 0.25) (layer "F.Cu") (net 19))
 (segment (start 81.7243 42.8457) (end 85.003 46.1244) (width 0.25) (layer "F.Cu") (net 19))
 (segment (start 76.9357 42.8457) (end 81.7243 42.8457) (width 0.25) (layer "F.Cu") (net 19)))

